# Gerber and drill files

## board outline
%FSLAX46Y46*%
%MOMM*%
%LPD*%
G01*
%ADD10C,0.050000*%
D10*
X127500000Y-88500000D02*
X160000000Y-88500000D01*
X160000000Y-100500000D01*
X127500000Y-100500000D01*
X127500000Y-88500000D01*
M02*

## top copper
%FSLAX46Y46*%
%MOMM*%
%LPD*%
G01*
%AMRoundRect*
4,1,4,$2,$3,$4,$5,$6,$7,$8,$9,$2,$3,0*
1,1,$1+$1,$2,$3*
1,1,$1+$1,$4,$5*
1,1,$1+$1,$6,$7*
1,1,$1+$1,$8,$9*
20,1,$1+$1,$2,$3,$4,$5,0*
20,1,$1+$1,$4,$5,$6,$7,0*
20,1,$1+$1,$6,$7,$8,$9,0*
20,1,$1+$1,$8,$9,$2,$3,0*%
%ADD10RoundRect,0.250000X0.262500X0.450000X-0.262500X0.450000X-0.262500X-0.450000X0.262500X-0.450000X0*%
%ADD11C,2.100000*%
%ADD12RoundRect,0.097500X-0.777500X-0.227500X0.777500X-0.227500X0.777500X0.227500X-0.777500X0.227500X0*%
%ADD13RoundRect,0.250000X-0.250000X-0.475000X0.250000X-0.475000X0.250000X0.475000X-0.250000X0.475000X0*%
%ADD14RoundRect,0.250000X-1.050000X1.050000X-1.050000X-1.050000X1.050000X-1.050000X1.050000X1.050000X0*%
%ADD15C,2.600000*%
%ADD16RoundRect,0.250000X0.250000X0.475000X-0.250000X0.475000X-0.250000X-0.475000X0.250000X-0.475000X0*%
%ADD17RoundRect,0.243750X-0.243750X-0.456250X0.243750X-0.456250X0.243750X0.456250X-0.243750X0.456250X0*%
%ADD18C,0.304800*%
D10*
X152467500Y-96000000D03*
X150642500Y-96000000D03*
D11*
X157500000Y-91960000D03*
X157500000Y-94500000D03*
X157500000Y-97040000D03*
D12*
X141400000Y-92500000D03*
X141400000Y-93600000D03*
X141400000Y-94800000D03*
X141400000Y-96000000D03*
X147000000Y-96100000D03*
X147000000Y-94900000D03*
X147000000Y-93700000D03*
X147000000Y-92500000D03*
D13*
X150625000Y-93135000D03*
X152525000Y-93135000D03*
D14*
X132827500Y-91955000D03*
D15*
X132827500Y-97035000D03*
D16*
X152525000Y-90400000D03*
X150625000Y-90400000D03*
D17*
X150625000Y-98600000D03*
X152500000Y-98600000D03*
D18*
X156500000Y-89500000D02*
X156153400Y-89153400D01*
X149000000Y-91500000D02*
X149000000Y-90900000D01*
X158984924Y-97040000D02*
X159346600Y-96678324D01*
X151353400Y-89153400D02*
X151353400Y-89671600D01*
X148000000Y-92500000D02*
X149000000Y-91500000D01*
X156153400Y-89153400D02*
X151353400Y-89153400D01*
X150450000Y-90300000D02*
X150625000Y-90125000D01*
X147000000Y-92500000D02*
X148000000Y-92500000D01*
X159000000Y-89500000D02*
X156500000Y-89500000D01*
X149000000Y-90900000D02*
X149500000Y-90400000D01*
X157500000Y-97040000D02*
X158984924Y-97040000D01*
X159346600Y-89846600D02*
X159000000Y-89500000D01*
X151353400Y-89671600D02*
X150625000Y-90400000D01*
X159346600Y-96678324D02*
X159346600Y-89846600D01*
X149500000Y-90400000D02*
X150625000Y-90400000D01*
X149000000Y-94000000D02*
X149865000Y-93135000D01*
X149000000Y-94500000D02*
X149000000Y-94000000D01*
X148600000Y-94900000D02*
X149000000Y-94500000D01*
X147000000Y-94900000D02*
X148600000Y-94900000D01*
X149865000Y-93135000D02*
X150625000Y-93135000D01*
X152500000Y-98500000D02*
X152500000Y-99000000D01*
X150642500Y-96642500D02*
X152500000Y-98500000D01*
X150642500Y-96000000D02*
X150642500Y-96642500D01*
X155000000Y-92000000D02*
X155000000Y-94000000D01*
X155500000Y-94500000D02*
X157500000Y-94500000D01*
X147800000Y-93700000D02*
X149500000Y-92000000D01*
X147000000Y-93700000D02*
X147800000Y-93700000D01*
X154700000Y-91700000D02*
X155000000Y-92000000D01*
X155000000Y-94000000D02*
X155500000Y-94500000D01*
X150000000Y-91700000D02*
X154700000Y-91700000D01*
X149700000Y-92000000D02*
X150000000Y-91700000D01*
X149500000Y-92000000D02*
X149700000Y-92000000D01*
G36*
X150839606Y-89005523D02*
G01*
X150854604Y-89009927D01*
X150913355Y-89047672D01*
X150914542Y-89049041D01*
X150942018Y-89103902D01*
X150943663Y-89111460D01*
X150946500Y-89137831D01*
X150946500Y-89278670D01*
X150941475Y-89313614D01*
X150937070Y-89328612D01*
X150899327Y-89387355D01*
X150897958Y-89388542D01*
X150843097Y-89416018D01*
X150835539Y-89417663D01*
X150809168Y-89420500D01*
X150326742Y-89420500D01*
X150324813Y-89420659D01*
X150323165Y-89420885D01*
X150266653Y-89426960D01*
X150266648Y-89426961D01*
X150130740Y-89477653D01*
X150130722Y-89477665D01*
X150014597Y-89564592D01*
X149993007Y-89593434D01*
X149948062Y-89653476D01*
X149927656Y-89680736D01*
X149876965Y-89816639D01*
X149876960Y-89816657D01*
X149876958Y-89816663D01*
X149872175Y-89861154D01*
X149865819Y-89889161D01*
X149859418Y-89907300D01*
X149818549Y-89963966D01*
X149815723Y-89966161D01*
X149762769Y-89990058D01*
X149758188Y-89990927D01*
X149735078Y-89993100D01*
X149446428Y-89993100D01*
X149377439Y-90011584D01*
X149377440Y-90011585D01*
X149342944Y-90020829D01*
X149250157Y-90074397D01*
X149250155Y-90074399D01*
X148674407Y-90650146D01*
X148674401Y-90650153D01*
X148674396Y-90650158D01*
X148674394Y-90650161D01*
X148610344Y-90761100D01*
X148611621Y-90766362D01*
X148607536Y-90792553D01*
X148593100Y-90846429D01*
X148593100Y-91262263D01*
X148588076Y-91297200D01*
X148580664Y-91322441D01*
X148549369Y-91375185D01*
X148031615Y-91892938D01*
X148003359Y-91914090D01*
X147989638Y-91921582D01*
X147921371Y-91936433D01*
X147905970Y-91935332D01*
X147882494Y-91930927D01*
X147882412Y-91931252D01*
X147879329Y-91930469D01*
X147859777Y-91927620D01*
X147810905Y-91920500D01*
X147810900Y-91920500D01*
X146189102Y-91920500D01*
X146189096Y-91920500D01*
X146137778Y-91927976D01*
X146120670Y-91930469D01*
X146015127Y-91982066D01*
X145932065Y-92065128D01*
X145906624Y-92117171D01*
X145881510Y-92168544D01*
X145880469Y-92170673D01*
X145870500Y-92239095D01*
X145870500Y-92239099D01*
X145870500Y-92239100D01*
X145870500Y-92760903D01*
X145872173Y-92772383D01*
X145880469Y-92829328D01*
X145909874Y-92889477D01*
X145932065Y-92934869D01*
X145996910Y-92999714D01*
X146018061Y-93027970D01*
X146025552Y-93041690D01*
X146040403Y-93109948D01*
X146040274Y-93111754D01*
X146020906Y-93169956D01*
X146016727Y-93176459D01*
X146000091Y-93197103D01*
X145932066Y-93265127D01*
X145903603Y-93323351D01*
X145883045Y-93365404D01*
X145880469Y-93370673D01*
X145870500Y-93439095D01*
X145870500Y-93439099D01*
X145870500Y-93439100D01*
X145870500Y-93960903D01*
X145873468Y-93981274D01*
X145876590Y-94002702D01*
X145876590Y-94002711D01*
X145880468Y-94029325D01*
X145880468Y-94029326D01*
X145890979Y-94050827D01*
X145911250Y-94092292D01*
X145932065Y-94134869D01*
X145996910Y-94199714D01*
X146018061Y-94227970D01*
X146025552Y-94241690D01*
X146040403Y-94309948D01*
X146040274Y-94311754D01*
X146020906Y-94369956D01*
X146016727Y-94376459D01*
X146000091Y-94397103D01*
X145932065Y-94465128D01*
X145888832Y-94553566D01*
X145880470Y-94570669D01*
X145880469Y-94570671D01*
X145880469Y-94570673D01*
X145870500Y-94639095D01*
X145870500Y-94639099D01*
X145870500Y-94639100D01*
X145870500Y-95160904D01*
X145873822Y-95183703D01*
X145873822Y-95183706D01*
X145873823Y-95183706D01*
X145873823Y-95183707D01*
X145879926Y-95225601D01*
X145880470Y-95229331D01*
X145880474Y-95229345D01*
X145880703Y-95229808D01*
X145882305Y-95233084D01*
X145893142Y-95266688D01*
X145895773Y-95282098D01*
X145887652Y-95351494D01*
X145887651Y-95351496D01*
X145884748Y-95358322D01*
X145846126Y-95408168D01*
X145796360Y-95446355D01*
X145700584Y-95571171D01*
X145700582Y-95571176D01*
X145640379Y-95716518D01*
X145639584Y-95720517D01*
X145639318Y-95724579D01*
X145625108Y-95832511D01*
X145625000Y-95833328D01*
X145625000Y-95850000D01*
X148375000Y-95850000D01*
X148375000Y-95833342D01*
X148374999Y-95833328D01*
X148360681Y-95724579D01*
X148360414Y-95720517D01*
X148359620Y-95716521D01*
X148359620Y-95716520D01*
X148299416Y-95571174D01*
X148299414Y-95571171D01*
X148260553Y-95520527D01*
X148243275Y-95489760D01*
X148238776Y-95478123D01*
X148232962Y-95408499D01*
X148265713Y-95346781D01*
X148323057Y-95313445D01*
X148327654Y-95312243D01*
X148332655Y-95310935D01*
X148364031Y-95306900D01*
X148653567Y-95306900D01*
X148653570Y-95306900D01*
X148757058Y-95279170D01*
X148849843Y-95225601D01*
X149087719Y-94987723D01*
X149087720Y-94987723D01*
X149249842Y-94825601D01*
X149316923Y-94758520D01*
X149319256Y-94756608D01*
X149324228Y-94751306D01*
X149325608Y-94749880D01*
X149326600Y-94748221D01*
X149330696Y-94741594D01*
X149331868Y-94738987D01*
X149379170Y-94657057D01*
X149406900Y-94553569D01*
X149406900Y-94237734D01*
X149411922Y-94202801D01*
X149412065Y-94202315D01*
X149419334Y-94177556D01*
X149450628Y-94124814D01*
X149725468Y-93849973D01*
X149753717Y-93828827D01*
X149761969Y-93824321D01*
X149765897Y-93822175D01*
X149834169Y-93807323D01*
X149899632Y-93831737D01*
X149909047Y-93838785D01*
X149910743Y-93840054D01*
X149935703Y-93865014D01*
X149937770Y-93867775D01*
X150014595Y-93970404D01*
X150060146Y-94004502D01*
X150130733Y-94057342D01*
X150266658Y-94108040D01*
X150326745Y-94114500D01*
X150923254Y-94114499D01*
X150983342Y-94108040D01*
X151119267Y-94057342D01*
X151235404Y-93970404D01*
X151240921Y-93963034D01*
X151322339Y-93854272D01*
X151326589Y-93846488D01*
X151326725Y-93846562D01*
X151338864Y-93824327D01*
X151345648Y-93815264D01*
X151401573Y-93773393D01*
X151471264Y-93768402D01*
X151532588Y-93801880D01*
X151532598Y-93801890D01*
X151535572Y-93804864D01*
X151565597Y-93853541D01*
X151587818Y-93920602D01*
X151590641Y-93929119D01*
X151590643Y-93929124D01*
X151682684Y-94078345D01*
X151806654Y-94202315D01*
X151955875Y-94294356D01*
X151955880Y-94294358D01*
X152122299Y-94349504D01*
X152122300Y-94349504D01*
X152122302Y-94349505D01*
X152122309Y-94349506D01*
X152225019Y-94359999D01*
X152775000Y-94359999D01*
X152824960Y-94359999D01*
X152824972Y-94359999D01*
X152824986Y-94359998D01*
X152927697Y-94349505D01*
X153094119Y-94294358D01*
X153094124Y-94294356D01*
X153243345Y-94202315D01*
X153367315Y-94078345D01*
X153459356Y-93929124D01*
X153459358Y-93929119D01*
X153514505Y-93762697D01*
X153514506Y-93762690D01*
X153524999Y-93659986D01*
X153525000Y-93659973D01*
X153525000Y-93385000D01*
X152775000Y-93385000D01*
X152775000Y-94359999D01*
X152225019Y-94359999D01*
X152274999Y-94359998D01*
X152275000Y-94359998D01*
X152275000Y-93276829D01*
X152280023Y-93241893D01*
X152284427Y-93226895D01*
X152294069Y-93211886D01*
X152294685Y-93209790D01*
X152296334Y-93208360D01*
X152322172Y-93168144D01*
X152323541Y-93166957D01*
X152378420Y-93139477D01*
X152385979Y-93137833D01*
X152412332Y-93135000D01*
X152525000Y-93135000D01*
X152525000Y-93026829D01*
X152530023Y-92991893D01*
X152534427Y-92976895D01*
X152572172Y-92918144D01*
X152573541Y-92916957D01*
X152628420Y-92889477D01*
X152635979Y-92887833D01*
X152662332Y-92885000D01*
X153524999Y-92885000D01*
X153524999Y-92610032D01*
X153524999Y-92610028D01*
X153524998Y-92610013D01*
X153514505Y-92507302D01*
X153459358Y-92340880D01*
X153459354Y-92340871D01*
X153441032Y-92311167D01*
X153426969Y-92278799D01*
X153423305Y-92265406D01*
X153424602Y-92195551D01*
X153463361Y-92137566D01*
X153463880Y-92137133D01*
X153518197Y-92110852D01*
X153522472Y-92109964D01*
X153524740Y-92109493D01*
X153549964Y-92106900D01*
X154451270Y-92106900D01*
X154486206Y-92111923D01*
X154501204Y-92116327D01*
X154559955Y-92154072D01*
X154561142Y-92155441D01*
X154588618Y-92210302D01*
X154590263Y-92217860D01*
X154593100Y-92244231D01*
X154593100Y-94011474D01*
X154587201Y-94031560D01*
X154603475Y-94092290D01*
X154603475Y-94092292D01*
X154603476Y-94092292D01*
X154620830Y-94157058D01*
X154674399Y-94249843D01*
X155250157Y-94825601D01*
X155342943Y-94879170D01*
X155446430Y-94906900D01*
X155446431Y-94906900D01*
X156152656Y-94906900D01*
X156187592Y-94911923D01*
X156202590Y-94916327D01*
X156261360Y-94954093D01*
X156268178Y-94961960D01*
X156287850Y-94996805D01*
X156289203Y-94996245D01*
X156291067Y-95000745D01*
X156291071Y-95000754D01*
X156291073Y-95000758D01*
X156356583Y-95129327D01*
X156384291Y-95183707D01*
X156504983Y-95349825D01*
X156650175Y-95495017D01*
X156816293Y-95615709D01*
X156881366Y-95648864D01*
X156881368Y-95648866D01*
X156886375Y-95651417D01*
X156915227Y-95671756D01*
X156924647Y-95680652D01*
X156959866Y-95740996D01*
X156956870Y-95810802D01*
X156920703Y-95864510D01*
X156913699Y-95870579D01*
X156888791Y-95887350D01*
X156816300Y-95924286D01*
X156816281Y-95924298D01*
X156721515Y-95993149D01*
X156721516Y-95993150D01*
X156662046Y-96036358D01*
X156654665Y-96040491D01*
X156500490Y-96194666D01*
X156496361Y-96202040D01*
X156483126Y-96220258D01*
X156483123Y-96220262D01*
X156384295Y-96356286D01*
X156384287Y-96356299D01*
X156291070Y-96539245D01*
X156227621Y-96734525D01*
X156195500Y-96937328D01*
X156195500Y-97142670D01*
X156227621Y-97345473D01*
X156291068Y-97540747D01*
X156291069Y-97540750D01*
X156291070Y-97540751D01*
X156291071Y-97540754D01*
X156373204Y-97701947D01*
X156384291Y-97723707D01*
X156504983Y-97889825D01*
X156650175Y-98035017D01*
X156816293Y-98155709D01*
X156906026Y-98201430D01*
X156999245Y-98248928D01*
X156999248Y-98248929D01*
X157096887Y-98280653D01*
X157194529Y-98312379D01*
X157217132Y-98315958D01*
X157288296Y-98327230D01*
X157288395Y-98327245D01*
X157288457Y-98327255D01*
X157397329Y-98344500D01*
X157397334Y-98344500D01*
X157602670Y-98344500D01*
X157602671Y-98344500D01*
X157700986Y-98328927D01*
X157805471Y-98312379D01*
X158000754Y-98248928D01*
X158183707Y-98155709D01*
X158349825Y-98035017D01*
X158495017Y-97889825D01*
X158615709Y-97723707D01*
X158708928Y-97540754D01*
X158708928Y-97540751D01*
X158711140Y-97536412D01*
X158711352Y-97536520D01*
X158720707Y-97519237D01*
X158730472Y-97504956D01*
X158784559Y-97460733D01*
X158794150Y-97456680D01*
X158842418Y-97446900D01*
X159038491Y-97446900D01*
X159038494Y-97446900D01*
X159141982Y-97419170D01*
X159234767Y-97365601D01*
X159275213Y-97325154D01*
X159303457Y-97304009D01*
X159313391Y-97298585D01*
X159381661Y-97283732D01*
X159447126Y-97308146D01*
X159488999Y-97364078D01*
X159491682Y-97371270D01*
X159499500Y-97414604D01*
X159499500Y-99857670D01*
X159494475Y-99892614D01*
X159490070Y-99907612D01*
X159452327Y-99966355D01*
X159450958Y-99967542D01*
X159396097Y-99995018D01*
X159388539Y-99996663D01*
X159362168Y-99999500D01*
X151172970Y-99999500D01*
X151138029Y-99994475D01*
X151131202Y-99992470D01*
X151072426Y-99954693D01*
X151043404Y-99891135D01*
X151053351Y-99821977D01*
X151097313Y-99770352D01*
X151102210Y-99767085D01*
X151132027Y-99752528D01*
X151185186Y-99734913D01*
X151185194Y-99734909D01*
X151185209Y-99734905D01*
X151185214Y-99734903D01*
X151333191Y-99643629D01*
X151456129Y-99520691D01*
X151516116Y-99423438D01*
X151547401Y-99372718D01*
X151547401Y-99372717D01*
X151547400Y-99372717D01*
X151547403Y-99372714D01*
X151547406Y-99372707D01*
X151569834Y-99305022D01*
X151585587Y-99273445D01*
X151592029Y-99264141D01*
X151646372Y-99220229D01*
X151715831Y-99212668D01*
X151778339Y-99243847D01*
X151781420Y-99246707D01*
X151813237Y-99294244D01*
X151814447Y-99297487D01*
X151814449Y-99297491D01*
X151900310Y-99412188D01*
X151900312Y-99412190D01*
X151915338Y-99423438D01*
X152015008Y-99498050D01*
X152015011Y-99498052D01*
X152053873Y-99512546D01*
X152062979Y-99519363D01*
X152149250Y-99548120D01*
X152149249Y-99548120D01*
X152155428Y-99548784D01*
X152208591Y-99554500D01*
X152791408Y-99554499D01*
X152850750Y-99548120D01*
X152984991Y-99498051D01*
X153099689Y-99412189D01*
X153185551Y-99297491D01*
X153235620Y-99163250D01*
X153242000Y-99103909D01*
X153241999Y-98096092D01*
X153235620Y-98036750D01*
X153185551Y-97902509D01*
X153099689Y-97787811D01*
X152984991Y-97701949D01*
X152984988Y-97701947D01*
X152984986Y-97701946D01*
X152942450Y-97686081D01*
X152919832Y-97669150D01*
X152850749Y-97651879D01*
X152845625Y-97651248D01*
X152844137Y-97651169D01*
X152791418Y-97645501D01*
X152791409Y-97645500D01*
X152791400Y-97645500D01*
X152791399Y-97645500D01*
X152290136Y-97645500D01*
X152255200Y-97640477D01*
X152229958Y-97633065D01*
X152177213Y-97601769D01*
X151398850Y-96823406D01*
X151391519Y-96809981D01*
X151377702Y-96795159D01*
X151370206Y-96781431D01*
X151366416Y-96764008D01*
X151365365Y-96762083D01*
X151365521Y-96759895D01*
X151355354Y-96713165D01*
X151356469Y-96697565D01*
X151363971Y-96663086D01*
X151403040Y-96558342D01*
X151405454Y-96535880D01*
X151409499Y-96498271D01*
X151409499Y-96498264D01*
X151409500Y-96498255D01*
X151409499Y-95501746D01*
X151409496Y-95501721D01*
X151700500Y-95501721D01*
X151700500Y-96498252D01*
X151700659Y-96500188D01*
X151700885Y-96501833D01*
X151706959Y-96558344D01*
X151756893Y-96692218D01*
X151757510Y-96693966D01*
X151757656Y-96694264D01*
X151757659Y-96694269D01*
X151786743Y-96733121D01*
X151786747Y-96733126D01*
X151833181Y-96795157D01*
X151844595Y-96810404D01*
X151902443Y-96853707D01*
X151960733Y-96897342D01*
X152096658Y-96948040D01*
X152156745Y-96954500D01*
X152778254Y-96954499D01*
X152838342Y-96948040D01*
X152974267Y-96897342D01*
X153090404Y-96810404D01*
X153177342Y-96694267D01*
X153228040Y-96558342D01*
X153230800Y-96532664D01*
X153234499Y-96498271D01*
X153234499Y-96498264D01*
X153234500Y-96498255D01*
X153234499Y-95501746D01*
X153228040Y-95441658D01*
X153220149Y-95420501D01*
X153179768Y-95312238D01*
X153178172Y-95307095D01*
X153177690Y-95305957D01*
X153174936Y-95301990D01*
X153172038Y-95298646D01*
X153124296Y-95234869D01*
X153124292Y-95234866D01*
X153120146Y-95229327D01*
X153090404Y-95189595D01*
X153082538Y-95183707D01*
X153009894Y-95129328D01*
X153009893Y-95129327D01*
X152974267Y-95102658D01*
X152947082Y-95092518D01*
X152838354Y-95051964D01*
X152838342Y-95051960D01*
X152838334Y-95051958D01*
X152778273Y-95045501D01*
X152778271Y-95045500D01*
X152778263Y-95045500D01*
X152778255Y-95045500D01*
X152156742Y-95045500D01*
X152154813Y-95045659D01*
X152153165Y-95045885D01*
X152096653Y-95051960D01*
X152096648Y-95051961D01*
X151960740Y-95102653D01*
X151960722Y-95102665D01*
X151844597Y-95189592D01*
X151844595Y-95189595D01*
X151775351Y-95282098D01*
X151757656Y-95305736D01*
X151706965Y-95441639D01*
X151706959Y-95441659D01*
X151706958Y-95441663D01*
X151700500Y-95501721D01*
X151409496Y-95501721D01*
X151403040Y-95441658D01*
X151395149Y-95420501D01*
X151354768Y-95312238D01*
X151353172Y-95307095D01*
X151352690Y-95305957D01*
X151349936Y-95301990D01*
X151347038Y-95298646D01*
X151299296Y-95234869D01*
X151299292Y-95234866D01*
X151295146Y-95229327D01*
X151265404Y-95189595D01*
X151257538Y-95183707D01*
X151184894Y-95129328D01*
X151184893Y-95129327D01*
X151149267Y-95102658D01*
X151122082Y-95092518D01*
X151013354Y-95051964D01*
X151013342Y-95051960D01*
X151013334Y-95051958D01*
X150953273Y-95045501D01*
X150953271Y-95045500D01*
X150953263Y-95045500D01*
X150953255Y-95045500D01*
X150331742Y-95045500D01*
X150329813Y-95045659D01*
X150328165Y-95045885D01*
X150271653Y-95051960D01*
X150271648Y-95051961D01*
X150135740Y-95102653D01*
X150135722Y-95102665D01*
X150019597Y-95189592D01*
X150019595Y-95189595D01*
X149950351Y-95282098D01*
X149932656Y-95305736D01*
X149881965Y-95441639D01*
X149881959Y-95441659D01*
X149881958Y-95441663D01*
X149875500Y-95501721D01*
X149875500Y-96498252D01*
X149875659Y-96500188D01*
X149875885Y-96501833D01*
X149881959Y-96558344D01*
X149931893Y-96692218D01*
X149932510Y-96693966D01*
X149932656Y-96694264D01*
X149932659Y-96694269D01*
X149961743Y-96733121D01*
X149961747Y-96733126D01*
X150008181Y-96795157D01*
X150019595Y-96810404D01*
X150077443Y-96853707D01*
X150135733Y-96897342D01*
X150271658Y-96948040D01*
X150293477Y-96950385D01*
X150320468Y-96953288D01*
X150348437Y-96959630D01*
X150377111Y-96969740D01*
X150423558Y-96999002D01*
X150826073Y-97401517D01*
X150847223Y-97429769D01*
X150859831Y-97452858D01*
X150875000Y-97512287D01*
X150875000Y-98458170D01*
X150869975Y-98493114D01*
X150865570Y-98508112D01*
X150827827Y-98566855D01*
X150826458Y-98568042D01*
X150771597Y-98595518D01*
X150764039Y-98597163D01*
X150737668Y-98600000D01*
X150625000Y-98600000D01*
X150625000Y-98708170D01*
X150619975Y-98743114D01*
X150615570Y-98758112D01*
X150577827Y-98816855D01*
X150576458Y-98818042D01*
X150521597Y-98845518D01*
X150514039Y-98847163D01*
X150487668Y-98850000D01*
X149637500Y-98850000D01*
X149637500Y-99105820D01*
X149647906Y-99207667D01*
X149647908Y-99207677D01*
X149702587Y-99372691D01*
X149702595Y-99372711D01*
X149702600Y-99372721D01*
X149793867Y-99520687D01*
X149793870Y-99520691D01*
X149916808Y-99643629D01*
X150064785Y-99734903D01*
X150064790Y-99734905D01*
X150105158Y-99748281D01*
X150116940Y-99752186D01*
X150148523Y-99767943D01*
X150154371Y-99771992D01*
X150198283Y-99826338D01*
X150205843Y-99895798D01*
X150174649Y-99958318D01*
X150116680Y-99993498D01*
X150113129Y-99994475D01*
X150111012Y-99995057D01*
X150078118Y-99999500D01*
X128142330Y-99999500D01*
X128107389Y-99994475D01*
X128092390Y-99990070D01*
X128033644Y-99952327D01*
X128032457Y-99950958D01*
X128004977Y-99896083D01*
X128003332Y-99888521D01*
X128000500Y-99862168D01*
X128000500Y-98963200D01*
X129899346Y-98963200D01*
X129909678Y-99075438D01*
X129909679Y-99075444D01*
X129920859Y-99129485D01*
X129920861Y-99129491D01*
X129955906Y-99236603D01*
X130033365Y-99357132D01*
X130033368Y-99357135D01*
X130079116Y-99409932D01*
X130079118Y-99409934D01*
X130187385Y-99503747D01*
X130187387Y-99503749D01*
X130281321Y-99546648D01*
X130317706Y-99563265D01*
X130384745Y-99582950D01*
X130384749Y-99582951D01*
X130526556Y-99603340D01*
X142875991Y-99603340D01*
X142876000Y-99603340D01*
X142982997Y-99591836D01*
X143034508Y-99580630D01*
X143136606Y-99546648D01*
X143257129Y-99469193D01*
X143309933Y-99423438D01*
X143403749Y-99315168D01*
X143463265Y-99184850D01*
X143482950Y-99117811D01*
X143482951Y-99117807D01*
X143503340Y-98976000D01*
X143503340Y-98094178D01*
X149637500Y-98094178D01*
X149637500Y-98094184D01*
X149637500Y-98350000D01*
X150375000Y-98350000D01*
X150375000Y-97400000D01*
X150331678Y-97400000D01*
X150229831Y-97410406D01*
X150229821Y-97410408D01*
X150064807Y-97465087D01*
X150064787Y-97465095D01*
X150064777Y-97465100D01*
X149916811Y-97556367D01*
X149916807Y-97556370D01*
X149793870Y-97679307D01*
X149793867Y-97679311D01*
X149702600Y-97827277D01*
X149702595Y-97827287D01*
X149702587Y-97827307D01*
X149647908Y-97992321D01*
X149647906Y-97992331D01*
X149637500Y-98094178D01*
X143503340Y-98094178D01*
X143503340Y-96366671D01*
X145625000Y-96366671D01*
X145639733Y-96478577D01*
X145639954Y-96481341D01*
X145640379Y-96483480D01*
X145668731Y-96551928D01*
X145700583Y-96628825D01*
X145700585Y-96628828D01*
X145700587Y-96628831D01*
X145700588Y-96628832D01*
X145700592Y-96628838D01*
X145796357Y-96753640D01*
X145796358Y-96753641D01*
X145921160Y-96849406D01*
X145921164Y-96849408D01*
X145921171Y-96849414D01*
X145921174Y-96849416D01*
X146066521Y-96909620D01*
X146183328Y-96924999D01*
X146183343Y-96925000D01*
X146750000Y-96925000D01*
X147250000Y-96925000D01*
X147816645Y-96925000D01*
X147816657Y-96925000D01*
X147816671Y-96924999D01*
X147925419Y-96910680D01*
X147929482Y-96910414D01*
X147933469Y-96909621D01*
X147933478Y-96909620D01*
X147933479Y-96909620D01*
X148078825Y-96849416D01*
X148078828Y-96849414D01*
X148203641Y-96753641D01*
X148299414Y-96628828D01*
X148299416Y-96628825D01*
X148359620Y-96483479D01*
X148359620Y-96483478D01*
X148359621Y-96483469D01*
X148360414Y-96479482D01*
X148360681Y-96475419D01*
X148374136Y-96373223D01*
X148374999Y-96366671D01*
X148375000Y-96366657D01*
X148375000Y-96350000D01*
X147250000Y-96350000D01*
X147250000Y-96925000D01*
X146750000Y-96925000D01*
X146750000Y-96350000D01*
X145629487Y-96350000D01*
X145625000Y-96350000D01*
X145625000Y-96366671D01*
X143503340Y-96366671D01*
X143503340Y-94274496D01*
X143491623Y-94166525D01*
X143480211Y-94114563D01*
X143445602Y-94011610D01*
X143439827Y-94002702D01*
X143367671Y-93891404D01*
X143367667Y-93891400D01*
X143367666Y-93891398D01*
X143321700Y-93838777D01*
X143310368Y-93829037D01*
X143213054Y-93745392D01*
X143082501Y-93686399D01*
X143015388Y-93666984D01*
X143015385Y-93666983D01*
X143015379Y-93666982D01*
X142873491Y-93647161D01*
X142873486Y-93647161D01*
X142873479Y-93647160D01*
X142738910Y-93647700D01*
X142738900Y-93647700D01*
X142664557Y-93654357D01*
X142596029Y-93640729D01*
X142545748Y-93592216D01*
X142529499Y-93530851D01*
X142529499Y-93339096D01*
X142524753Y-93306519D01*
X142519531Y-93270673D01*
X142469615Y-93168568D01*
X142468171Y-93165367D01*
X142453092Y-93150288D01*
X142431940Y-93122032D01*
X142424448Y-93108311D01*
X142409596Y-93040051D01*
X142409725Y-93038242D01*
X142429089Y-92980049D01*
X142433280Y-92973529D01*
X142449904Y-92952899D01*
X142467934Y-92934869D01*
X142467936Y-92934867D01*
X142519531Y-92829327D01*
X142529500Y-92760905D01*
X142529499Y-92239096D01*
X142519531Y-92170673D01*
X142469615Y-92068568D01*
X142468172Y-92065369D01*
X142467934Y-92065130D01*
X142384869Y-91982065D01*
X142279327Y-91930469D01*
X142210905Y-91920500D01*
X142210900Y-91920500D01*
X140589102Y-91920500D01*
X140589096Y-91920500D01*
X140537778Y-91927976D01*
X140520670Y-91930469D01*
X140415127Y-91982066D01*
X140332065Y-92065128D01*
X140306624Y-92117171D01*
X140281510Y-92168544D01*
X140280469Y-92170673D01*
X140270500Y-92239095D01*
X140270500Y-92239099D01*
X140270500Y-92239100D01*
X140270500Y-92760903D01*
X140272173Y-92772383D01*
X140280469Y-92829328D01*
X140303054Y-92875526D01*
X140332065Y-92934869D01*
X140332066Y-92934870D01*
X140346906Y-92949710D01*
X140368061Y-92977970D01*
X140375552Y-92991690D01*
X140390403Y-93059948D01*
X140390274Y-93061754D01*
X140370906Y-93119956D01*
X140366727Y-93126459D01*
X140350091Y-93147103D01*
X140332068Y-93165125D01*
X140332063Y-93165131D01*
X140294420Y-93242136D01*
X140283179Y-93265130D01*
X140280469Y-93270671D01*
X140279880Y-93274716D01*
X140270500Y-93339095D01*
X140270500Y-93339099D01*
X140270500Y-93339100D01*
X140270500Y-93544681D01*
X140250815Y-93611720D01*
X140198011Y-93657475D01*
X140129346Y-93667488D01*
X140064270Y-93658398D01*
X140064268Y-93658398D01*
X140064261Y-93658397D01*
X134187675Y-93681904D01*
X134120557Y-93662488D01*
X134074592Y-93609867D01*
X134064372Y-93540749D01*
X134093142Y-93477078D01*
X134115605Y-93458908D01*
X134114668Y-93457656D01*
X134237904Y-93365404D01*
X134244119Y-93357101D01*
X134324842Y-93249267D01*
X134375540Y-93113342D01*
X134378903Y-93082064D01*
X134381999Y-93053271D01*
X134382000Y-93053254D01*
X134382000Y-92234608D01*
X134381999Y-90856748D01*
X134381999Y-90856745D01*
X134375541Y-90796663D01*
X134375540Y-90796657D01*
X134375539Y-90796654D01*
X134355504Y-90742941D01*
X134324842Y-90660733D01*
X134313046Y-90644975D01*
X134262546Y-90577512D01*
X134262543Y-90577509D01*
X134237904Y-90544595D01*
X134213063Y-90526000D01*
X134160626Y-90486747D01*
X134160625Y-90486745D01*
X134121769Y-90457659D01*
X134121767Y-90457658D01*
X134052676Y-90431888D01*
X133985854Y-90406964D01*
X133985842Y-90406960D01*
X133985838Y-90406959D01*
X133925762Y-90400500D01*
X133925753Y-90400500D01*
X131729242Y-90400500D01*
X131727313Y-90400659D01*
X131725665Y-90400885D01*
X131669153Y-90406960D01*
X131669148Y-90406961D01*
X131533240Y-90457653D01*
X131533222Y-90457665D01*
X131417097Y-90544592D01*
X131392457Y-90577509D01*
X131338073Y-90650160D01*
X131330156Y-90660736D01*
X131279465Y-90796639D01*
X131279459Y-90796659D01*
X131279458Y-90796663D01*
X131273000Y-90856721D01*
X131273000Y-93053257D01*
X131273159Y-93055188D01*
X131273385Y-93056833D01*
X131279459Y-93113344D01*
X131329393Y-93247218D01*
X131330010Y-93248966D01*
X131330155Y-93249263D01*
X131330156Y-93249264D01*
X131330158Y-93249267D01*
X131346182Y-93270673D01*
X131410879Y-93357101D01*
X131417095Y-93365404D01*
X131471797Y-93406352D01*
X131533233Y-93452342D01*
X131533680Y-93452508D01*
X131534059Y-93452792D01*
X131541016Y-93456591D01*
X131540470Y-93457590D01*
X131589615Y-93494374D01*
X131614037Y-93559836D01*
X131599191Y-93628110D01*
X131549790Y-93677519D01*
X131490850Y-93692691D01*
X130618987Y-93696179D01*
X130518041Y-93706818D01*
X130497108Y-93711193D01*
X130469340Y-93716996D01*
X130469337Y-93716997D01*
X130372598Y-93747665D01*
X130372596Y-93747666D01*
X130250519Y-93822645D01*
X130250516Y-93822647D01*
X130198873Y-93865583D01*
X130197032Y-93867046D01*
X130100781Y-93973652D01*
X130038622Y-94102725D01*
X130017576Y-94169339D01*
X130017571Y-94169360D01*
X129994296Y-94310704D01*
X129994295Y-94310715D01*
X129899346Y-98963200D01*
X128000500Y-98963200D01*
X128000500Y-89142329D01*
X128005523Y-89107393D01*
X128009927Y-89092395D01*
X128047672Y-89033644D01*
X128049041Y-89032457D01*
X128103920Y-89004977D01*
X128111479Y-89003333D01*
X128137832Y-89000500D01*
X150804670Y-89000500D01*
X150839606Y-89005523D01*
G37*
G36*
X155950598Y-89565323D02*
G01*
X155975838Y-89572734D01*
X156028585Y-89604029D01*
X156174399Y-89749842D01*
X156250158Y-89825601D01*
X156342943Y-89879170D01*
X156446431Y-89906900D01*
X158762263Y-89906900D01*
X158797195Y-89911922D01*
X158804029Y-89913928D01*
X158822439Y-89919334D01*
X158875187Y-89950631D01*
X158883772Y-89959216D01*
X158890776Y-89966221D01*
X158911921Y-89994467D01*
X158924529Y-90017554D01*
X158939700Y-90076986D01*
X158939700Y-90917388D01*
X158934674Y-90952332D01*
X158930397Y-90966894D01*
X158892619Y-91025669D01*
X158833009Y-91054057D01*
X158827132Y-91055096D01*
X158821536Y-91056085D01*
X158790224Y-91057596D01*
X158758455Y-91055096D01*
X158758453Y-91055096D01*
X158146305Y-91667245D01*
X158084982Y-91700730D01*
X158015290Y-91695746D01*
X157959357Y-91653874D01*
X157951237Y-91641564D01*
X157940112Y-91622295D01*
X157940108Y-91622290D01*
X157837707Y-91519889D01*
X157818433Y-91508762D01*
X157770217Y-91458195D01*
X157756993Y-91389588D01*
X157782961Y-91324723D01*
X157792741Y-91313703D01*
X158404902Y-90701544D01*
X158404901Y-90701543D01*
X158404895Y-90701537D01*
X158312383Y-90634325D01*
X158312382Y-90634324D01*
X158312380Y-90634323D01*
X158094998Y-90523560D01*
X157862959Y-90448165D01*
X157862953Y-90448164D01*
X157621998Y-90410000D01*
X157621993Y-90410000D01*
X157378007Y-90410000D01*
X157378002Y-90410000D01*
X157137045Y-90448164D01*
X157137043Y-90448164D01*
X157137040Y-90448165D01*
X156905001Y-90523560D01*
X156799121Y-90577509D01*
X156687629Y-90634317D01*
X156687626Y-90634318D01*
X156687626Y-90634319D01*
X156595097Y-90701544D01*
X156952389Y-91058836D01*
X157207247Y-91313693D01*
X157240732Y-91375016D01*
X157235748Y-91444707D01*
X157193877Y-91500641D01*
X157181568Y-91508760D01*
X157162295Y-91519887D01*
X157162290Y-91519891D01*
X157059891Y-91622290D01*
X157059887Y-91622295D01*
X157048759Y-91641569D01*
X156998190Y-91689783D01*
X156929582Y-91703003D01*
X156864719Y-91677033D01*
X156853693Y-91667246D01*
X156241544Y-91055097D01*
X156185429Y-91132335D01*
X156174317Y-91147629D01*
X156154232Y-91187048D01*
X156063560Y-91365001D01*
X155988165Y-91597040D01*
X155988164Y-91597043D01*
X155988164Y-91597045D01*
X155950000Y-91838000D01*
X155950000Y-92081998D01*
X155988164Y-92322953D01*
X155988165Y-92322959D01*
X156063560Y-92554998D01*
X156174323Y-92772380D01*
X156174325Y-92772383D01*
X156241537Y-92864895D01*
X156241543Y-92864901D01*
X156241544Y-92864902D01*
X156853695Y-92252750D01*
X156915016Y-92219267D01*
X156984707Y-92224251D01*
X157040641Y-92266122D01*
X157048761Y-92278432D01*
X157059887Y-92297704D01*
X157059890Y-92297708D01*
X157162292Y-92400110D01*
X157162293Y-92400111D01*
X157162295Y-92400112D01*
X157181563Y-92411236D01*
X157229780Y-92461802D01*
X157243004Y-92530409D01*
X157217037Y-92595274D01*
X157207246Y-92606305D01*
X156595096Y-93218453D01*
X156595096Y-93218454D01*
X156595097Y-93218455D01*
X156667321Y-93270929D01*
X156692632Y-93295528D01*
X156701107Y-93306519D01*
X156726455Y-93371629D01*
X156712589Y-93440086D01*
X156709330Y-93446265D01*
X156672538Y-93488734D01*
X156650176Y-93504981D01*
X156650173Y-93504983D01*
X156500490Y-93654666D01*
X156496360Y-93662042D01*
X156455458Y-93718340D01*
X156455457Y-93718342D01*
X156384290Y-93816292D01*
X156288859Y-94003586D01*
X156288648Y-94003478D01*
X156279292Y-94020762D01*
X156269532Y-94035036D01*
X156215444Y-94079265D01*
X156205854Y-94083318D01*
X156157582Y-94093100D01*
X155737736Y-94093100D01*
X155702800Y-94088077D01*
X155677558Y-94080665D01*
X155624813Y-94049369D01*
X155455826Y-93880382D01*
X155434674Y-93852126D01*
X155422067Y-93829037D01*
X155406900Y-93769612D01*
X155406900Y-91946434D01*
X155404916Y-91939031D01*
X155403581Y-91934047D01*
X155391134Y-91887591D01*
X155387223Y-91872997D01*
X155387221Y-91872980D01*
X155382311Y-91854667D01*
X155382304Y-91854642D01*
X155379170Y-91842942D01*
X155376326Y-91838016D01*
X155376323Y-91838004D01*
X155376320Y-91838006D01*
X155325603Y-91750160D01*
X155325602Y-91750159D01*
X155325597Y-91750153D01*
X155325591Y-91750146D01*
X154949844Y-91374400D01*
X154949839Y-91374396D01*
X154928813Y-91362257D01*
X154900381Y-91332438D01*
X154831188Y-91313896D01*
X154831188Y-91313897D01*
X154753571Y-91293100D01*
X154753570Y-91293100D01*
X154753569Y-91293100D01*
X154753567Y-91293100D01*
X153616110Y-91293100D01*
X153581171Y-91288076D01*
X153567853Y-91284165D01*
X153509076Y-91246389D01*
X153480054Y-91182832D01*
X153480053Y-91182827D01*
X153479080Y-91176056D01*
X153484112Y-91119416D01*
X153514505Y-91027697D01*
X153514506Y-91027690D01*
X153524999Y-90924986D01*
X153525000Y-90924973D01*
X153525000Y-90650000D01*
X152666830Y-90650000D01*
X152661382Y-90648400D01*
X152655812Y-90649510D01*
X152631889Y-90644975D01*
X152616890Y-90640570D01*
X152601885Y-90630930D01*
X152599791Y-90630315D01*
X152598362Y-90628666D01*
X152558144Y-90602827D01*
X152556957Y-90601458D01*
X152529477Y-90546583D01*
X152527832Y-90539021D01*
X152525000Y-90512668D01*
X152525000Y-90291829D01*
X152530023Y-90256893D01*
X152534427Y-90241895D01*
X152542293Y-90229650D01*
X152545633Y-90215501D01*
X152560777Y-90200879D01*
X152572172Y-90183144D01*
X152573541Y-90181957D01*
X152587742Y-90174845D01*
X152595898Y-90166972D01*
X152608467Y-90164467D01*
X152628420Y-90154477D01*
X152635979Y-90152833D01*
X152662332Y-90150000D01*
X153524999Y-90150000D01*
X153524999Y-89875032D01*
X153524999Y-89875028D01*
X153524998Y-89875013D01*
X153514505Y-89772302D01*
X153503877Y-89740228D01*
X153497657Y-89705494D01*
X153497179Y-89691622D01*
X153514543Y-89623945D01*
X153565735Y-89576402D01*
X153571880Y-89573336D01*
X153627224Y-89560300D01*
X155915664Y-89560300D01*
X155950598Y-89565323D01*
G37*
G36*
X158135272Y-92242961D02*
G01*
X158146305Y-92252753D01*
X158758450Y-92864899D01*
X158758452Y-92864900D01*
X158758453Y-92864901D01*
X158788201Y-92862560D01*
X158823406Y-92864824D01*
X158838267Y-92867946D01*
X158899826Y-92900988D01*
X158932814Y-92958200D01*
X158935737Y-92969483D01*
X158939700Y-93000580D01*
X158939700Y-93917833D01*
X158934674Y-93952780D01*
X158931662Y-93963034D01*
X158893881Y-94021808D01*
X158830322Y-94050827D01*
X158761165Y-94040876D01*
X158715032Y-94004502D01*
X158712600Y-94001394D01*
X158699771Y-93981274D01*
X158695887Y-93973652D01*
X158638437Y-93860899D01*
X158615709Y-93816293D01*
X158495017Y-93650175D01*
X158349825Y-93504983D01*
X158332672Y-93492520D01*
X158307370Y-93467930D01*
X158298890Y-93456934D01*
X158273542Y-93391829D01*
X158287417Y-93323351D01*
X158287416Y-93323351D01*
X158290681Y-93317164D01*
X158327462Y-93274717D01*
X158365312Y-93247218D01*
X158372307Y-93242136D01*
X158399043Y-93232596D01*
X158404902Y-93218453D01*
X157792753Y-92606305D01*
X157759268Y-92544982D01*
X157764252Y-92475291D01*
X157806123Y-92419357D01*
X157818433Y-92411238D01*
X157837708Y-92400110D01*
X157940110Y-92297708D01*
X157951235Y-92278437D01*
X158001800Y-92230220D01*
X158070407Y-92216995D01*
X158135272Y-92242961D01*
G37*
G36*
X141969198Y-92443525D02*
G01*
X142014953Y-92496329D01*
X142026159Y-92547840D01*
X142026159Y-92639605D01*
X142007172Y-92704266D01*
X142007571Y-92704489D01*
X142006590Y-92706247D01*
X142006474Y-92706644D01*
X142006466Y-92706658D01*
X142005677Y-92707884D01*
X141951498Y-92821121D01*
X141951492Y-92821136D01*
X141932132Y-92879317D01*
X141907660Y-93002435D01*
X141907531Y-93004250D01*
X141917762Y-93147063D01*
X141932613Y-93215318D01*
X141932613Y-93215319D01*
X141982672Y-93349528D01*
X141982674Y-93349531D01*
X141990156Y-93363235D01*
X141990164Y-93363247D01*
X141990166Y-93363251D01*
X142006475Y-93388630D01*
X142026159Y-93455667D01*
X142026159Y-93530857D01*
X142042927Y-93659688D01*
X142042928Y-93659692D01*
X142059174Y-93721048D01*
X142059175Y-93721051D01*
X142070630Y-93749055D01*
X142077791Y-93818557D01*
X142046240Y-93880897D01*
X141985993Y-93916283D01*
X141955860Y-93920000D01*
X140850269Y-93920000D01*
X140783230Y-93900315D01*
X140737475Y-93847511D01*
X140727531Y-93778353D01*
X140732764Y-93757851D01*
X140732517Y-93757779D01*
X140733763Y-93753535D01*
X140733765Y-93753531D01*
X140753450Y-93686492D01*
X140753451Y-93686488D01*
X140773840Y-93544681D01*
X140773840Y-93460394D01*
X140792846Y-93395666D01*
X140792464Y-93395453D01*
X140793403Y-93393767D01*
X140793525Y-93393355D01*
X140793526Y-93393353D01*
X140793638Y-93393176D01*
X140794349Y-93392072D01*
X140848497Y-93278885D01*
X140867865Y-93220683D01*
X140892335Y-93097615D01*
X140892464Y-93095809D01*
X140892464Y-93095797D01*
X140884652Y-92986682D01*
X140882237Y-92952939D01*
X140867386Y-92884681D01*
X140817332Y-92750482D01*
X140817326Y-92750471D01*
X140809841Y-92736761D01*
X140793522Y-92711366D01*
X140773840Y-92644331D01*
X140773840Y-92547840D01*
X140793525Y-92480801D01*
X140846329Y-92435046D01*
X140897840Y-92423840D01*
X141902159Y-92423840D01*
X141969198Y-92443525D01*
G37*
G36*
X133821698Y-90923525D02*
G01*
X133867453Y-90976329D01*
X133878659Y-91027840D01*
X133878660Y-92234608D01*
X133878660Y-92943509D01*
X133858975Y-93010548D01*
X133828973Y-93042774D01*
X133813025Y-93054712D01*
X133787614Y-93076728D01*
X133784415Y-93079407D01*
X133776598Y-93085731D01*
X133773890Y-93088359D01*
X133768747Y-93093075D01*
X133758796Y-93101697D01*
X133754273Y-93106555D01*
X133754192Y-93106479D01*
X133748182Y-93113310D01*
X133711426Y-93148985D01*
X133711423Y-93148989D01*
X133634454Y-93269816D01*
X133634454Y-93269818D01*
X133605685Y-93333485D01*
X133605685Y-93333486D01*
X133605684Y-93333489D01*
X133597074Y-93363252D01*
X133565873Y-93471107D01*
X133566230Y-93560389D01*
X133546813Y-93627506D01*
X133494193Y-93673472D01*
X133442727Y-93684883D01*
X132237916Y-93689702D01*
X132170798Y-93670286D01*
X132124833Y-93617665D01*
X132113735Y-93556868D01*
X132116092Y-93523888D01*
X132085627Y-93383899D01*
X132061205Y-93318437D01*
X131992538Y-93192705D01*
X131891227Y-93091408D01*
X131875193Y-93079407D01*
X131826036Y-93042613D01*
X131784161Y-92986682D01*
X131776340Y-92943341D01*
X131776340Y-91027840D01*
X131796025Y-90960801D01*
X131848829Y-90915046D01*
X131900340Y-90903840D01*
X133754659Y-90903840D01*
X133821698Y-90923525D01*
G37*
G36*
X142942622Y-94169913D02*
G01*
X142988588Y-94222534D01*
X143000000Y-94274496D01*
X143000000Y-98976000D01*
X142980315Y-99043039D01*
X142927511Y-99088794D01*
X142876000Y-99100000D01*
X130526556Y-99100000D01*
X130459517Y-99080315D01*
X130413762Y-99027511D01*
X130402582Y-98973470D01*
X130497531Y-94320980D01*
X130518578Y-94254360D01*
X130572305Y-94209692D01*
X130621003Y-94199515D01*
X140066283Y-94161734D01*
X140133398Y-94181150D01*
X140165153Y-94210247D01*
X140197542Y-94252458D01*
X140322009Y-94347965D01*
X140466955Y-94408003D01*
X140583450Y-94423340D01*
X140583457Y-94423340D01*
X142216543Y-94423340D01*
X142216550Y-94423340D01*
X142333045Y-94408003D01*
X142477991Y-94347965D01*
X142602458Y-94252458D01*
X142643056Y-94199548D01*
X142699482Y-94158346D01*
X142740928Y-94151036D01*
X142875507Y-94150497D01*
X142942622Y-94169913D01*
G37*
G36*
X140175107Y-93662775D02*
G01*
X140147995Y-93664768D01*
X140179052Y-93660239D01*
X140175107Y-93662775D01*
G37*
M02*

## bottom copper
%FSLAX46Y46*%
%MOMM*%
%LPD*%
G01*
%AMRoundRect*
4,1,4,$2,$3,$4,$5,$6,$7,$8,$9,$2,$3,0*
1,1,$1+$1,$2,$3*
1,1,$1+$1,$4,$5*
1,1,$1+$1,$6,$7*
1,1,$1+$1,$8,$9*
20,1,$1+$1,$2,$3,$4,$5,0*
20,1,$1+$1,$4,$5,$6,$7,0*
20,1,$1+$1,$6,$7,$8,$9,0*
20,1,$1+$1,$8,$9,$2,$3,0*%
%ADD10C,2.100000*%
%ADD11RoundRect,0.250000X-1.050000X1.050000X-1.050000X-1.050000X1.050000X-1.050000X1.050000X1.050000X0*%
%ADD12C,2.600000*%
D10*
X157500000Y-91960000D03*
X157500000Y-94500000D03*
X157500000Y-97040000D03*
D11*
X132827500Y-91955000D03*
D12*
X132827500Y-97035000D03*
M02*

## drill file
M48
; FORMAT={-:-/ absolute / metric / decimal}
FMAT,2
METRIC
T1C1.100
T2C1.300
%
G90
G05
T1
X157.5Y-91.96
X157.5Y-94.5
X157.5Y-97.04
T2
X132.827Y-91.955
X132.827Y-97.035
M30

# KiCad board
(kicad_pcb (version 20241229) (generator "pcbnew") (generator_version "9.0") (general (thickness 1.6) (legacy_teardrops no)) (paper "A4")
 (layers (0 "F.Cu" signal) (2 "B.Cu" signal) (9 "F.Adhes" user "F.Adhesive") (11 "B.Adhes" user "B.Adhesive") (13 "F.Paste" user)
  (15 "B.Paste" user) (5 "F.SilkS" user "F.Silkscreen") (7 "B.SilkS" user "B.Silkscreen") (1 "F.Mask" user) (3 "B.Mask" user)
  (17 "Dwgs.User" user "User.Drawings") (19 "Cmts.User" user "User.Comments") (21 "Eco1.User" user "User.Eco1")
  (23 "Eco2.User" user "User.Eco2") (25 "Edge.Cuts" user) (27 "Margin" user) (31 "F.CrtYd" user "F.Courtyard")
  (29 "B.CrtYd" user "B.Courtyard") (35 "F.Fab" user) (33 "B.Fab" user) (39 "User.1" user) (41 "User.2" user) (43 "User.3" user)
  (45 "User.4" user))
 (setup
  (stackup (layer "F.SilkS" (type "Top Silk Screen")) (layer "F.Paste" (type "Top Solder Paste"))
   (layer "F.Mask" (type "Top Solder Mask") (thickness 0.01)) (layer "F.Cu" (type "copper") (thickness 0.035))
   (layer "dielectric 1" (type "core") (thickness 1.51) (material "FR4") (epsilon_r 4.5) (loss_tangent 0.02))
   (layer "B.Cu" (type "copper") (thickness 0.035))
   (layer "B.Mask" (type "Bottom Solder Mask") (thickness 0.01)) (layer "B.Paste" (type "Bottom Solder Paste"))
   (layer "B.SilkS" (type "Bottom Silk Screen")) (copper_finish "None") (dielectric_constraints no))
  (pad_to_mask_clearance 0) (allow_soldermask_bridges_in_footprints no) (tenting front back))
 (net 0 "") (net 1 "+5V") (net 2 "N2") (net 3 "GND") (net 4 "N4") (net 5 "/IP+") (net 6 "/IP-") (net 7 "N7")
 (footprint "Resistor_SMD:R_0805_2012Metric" (layer "F.Cu") (at 151.555 96 180)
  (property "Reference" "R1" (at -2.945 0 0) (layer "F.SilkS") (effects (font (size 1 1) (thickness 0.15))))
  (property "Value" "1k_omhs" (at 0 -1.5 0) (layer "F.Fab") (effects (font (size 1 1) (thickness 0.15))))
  (pad "1" smd roundrect (at -0.9125 0 180) (size 1.025 1.4) (layers "F.Cu" "F.Mask" "F.Paste") (roundrect_rratio 0.243902) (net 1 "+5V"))
  (pad "2" smd roundrect (at 0.9125 0 180) (size 1.025 1.4) (layers "F.Cu" "F.Mask" "F.Paste") (roundrect_rratio 0.243902) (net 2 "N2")))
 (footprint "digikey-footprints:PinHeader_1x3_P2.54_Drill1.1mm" (layer "F.Cu") (at 157.5 91.96 -90)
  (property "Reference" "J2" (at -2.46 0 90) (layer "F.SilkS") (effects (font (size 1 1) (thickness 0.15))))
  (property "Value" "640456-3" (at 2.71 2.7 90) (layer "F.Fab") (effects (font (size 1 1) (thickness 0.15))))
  (pad "1" thru_hole circle (at 0 0 270) (size 2.1 2.1) (drill 1.1) (layers "*.Cu" "*.Mask") (remove_unused_layers no) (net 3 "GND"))
  (pad "2" thru_hole circle (at 2.54 0 270) (size 2.1 2.1) (drill 1.1) (layers "*.Cu" "*.Mask") (remove_unused_layers no) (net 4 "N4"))
  (pad "3" thru_hole circle (at 5.08 0 270) (size 2.1 2.1) (drill 1.1) (layers "*.Cu" "*.Mask") (remove_unused_layers no) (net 1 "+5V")))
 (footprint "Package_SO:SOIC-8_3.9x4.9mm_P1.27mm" (layer "F.Cu") (at 147 92.5)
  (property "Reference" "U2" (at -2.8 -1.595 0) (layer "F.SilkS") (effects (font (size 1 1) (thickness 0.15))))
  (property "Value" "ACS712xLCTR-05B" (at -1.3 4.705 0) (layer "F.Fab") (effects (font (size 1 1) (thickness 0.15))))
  (pad "1" smd roundrect (at -5.6 0) (size 1.75 0.65) (layers "F.Cu" "F.Mask" "F.Paste") (roundrect_rratio 0.15) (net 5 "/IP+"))
  (pad "2" smd roundrect (at -5.6 1.1) (size 1.75 0.65) (layers "F.Cu" "F.Mask" "F.Paste") (roundrect_rratio 0.15) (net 5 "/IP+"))
  (pad "3" smd roundrect (at -5.6 2.3) (size 1.75 0.65) (layers "F.Cu" "F.Mask" "F.Paste") (roundrect_rratio 0.15) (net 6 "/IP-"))
  (pad "4" smd roundrect (at -5.6 3.5) (size 1.75 0.65) (layers "F.Cu" "F.Mask" "F.Paste") (roundrect_rratio 0.15) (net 6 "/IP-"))
  (pad "5" smd roundrect (at 0 3.6) (size 1.75 0.65) (layers "F.Cu" "F.Mask" "F.Paste") (roundrect_rratio 0.15) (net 3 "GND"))
  (pad "6" smd roundrect (at 0 2.4) (size 1.75 0.65) (layers "F.Cu" "F.Mask" "F.Paste") (roundrect_rratio 0.15) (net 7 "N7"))
  (pad "7" smd roundrect (at 0 1.2) (size 1.75 0.65) (layers "F.Cu" "F.Mask" "F.Paste") (roundrect_rratio 0.15) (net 4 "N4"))
  (pad "8" smd roundrect (at 0 0) (size 1.75 0.65) (layers "F.Cu" "F.Mask" "F.Paste") (roundrect_rratio 0.15) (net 1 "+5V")))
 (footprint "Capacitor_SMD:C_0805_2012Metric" (layer "F.Cu") (at 151.575 93.135)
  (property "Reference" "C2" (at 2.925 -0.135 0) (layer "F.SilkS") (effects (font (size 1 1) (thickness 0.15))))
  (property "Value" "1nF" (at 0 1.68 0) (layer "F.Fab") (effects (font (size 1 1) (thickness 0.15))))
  (pad "1" smd roundrect (at -0.95 0) (size 1 1.45) (layers "F.Cu" "F.Mask" "F.Paste") (roundrect_rratio 0.25) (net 7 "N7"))
  (pad "2" smd roundrect (at 0.95 0) (size 1 1.45) (layers "F.Cu" "F.Mask" "F.Paste") (roundrect_rratio 0.25) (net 3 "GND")))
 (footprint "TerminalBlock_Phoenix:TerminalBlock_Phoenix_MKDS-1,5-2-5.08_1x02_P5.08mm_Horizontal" (layer "F.Cu") (at 132.8275 91.955 -90)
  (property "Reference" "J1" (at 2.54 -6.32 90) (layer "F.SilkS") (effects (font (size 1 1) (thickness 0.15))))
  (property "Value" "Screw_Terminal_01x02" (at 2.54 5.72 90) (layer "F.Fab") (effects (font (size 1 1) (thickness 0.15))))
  (pad "1" thru_hole roundrect (at 0 0 270) (size 2.6 2.6) (drill 1.3) (layers "*.Cu" "*.Mask") (remove_unused_layers no)
   (roundrect_rratio 0.096154) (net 5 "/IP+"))
  (pad "2" thru_hole circle (at 5.08 0 270) (size 2.6 2.6) (drill 1.3) (layers "*.Cu" "*.Mask") (remove_unused_layers no) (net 6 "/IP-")))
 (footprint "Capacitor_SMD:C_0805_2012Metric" (layer "F.Cu") (at 151.575 90.4 180)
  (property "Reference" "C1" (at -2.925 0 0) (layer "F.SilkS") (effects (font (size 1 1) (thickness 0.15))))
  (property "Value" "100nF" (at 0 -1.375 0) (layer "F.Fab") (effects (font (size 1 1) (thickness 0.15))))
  (pad "1" smd roundrect (at -0.95 0 180) (size 1 1.45) (layers "F.Cu" "F.Mask" "F.Paste") (roundrect_rratio 0.25) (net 3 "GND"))
  (pad "2" smd roundrect (at 0.95 0 180) (size 1 1.45) (layers "F.Cu" "F.Mask" "F.Paste") (roundrect_rratio 0.25) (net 1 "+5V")))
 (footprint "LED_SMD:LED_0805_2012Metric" (layer "F.Cu") (at 151.5625 98.6)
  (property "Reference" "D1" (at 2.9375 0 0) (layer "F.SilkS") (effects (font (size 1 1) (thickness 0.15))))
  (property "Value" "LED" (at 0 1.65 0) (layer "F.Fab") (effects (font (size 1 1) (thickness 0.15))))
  (pad "1" smd roundrect (at -0.9375 0) (size 0.975 1.4) (layers "F.Cu" "F.Mask" "F.Paste") (roundrect_rratio 0.25) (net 3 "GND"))
  (pad "2" smd roundrect (at 0.9375 0) (size 0.975 1.4) (layers "F.Cu" "F.Mask" "F.Paste") (roundrect_rratio 0.25) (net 2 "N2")))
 (gr_rect (start 127.5 88.5) (end 160 100.5) (stroke (width 0.05) (type default)) (fill no) (layer "Edge.Cuts"))
 (segment (start 156.5 89.5) (end 156.1534 89.1534) (width 0.3048) (layer "F.Cu") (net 1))
 (segment (start 149 91.5) (end 149 90.9) (width 0.3048) (layer "F.Cu") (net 1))
 (segment (start 158.984924 97.04) (end 159.3466 96.678324) (width 0.3048) (layer "F.Cu") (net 1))
 (segment (start 151.3534 89.1534) (end 151.3534 89.6716) (width 0.3048) (layer "F.Cu") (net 1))
 (segment (start 148 92.5) (end 149 91.5) (width 0.3048) (layer "F.Cu") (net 1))
 (segment (start 156.1534 89.1534) (end 151.3534 89.1534) (width 0.3048) (layer "F.Cu") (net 1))
 (segment (start 150.45 90.3) (end 150.625 90.125) (width 0.3048) (layer "F.Cu") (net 1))
 (segment (start 147 92.5) (end 148 92.5) (width 0.3048) (layer "F.Cu") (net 1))
 (segment (start 159 89.5) (end 156.5 89.5) (width 0.3048) (layer "F.Cu") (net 1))
 (segment (start 149 90.9) (end 149.5 90.4) (width 0.3048) (layer "F.Cu") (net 1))
 (segment (start 157.5 97.04) (end 158.984924 97.04) (width 0.3048) (layer "F.Cu") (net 1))
 (segment (start 159.3466 89.8466) (end 159 89.5) (width 0.3048) (layer "F.Cu") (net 1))
 (segment (start 151.3534 89.6716) (end 150.625 90.4) (width 0.3048) (layer "F.Cu") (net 1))
 (segment (start 159.3466 96.678324) (end 159.3466 89.8466) (width 0.3048) (layer "F.Cu") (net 1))
 (segment (start 149.5 90.4) (end 150.625 90.4) (width 0.3048) (layer "F.Cu") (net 1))
 (segment (start 149 94) (end 149.865 93.135) (width 0.3048) (layer "F.Cu") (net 7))
 (segment (start 149 94.5) (end 149 94) (width 0.3048) (layer "F.Cu") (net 7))
 (segment (start 148.6 94.9) (end 149 94.5) (width 0.3048) (layer "F.Cu") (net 7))
 (segment (start 147 94.9) (end 148.6 94.9) (width 0.3048) (layer "F.Cu") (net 7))
 (segment (start 149.865 93.135) (end 150.625 93.135) (width 0.3048) (layer "F.Cu") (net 7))
 (segment (start 152.5 98.5) (end 152.5 99) (width 0.3048) (layer "F.Cu") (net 2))
 (segment (start 150.6425 96.6425) (end 152.5 98.5) (width 0.3048) (layer "F.Cu") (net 2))
 (segment (start 150.6425 96) (end 150.6425 96.6425) (width 0.3048) (layer "F.Cu") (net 2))
 (segment (start 155 92) (end 155 94) (width 0.3048) (layer "F.Cu") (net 4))
 (segment (start 155.5 94.5) (end 157.5 94.5) (width 0.3048) (layer "F.Cu") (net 4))
 (segment (start 147.8 93.7) (end 149.5 92) (width 0.3048) (layer "F.Cu") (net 4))
 (segment (start 147 93.7) (end 147.8 93.7) (width 0.3048) (layer "F.Cu") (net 4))
 (segment (start 154.7 91.7) (end 155 92) (width 0.3048) (layer "F.Cu") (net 4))
 (segment (start 155 94) (end 155.5 94.5) (width 0.3048) (layer "F.Cu") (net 4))
 (segment (start 150 91.7) (end 154.7 91.7) (width 0.3048) (layer "F.Cu") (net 4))
 (segment (start 149.7 92) (end 150 91.7) (width 0.3048) (layer "F.Cu") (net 4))
 (segment (start 149.5 92) (end 149.7 92) (width 0.3048) (layer "F.Cu") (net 4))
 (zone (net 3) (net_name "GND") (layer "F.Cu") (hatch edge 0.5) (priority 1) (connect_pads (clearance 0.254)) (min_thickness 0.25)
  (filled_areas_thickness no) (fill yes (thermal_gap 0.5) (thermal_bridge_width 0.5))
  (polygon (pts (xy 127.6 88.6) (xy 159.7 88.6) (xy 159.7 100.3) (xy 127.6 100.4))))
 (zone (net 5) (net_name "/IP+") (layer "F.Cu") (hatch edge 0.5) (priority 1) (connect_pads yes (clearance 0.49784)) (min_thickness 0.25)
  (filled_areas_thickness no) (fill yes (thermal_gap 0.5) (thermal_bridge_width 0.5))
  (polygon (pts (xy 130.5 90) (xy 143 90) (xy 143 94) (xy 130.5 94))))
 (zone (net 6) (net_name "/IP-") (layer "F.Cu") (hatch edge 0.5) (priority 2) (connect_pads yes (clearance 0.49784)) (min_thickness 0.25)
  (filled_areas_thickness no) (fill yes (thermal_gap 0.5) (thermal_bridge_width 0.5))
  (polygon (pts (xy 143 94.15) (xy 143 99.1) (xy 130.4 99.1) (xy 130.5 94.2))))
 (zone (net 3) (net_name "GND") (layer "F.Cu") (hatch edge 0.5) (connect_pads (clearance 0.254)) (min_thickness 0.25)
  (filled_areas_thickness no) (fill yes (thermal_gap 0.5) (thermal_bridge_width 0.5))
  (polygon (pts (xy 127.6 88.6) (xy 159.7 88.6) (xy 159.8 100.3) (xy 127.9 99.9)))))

